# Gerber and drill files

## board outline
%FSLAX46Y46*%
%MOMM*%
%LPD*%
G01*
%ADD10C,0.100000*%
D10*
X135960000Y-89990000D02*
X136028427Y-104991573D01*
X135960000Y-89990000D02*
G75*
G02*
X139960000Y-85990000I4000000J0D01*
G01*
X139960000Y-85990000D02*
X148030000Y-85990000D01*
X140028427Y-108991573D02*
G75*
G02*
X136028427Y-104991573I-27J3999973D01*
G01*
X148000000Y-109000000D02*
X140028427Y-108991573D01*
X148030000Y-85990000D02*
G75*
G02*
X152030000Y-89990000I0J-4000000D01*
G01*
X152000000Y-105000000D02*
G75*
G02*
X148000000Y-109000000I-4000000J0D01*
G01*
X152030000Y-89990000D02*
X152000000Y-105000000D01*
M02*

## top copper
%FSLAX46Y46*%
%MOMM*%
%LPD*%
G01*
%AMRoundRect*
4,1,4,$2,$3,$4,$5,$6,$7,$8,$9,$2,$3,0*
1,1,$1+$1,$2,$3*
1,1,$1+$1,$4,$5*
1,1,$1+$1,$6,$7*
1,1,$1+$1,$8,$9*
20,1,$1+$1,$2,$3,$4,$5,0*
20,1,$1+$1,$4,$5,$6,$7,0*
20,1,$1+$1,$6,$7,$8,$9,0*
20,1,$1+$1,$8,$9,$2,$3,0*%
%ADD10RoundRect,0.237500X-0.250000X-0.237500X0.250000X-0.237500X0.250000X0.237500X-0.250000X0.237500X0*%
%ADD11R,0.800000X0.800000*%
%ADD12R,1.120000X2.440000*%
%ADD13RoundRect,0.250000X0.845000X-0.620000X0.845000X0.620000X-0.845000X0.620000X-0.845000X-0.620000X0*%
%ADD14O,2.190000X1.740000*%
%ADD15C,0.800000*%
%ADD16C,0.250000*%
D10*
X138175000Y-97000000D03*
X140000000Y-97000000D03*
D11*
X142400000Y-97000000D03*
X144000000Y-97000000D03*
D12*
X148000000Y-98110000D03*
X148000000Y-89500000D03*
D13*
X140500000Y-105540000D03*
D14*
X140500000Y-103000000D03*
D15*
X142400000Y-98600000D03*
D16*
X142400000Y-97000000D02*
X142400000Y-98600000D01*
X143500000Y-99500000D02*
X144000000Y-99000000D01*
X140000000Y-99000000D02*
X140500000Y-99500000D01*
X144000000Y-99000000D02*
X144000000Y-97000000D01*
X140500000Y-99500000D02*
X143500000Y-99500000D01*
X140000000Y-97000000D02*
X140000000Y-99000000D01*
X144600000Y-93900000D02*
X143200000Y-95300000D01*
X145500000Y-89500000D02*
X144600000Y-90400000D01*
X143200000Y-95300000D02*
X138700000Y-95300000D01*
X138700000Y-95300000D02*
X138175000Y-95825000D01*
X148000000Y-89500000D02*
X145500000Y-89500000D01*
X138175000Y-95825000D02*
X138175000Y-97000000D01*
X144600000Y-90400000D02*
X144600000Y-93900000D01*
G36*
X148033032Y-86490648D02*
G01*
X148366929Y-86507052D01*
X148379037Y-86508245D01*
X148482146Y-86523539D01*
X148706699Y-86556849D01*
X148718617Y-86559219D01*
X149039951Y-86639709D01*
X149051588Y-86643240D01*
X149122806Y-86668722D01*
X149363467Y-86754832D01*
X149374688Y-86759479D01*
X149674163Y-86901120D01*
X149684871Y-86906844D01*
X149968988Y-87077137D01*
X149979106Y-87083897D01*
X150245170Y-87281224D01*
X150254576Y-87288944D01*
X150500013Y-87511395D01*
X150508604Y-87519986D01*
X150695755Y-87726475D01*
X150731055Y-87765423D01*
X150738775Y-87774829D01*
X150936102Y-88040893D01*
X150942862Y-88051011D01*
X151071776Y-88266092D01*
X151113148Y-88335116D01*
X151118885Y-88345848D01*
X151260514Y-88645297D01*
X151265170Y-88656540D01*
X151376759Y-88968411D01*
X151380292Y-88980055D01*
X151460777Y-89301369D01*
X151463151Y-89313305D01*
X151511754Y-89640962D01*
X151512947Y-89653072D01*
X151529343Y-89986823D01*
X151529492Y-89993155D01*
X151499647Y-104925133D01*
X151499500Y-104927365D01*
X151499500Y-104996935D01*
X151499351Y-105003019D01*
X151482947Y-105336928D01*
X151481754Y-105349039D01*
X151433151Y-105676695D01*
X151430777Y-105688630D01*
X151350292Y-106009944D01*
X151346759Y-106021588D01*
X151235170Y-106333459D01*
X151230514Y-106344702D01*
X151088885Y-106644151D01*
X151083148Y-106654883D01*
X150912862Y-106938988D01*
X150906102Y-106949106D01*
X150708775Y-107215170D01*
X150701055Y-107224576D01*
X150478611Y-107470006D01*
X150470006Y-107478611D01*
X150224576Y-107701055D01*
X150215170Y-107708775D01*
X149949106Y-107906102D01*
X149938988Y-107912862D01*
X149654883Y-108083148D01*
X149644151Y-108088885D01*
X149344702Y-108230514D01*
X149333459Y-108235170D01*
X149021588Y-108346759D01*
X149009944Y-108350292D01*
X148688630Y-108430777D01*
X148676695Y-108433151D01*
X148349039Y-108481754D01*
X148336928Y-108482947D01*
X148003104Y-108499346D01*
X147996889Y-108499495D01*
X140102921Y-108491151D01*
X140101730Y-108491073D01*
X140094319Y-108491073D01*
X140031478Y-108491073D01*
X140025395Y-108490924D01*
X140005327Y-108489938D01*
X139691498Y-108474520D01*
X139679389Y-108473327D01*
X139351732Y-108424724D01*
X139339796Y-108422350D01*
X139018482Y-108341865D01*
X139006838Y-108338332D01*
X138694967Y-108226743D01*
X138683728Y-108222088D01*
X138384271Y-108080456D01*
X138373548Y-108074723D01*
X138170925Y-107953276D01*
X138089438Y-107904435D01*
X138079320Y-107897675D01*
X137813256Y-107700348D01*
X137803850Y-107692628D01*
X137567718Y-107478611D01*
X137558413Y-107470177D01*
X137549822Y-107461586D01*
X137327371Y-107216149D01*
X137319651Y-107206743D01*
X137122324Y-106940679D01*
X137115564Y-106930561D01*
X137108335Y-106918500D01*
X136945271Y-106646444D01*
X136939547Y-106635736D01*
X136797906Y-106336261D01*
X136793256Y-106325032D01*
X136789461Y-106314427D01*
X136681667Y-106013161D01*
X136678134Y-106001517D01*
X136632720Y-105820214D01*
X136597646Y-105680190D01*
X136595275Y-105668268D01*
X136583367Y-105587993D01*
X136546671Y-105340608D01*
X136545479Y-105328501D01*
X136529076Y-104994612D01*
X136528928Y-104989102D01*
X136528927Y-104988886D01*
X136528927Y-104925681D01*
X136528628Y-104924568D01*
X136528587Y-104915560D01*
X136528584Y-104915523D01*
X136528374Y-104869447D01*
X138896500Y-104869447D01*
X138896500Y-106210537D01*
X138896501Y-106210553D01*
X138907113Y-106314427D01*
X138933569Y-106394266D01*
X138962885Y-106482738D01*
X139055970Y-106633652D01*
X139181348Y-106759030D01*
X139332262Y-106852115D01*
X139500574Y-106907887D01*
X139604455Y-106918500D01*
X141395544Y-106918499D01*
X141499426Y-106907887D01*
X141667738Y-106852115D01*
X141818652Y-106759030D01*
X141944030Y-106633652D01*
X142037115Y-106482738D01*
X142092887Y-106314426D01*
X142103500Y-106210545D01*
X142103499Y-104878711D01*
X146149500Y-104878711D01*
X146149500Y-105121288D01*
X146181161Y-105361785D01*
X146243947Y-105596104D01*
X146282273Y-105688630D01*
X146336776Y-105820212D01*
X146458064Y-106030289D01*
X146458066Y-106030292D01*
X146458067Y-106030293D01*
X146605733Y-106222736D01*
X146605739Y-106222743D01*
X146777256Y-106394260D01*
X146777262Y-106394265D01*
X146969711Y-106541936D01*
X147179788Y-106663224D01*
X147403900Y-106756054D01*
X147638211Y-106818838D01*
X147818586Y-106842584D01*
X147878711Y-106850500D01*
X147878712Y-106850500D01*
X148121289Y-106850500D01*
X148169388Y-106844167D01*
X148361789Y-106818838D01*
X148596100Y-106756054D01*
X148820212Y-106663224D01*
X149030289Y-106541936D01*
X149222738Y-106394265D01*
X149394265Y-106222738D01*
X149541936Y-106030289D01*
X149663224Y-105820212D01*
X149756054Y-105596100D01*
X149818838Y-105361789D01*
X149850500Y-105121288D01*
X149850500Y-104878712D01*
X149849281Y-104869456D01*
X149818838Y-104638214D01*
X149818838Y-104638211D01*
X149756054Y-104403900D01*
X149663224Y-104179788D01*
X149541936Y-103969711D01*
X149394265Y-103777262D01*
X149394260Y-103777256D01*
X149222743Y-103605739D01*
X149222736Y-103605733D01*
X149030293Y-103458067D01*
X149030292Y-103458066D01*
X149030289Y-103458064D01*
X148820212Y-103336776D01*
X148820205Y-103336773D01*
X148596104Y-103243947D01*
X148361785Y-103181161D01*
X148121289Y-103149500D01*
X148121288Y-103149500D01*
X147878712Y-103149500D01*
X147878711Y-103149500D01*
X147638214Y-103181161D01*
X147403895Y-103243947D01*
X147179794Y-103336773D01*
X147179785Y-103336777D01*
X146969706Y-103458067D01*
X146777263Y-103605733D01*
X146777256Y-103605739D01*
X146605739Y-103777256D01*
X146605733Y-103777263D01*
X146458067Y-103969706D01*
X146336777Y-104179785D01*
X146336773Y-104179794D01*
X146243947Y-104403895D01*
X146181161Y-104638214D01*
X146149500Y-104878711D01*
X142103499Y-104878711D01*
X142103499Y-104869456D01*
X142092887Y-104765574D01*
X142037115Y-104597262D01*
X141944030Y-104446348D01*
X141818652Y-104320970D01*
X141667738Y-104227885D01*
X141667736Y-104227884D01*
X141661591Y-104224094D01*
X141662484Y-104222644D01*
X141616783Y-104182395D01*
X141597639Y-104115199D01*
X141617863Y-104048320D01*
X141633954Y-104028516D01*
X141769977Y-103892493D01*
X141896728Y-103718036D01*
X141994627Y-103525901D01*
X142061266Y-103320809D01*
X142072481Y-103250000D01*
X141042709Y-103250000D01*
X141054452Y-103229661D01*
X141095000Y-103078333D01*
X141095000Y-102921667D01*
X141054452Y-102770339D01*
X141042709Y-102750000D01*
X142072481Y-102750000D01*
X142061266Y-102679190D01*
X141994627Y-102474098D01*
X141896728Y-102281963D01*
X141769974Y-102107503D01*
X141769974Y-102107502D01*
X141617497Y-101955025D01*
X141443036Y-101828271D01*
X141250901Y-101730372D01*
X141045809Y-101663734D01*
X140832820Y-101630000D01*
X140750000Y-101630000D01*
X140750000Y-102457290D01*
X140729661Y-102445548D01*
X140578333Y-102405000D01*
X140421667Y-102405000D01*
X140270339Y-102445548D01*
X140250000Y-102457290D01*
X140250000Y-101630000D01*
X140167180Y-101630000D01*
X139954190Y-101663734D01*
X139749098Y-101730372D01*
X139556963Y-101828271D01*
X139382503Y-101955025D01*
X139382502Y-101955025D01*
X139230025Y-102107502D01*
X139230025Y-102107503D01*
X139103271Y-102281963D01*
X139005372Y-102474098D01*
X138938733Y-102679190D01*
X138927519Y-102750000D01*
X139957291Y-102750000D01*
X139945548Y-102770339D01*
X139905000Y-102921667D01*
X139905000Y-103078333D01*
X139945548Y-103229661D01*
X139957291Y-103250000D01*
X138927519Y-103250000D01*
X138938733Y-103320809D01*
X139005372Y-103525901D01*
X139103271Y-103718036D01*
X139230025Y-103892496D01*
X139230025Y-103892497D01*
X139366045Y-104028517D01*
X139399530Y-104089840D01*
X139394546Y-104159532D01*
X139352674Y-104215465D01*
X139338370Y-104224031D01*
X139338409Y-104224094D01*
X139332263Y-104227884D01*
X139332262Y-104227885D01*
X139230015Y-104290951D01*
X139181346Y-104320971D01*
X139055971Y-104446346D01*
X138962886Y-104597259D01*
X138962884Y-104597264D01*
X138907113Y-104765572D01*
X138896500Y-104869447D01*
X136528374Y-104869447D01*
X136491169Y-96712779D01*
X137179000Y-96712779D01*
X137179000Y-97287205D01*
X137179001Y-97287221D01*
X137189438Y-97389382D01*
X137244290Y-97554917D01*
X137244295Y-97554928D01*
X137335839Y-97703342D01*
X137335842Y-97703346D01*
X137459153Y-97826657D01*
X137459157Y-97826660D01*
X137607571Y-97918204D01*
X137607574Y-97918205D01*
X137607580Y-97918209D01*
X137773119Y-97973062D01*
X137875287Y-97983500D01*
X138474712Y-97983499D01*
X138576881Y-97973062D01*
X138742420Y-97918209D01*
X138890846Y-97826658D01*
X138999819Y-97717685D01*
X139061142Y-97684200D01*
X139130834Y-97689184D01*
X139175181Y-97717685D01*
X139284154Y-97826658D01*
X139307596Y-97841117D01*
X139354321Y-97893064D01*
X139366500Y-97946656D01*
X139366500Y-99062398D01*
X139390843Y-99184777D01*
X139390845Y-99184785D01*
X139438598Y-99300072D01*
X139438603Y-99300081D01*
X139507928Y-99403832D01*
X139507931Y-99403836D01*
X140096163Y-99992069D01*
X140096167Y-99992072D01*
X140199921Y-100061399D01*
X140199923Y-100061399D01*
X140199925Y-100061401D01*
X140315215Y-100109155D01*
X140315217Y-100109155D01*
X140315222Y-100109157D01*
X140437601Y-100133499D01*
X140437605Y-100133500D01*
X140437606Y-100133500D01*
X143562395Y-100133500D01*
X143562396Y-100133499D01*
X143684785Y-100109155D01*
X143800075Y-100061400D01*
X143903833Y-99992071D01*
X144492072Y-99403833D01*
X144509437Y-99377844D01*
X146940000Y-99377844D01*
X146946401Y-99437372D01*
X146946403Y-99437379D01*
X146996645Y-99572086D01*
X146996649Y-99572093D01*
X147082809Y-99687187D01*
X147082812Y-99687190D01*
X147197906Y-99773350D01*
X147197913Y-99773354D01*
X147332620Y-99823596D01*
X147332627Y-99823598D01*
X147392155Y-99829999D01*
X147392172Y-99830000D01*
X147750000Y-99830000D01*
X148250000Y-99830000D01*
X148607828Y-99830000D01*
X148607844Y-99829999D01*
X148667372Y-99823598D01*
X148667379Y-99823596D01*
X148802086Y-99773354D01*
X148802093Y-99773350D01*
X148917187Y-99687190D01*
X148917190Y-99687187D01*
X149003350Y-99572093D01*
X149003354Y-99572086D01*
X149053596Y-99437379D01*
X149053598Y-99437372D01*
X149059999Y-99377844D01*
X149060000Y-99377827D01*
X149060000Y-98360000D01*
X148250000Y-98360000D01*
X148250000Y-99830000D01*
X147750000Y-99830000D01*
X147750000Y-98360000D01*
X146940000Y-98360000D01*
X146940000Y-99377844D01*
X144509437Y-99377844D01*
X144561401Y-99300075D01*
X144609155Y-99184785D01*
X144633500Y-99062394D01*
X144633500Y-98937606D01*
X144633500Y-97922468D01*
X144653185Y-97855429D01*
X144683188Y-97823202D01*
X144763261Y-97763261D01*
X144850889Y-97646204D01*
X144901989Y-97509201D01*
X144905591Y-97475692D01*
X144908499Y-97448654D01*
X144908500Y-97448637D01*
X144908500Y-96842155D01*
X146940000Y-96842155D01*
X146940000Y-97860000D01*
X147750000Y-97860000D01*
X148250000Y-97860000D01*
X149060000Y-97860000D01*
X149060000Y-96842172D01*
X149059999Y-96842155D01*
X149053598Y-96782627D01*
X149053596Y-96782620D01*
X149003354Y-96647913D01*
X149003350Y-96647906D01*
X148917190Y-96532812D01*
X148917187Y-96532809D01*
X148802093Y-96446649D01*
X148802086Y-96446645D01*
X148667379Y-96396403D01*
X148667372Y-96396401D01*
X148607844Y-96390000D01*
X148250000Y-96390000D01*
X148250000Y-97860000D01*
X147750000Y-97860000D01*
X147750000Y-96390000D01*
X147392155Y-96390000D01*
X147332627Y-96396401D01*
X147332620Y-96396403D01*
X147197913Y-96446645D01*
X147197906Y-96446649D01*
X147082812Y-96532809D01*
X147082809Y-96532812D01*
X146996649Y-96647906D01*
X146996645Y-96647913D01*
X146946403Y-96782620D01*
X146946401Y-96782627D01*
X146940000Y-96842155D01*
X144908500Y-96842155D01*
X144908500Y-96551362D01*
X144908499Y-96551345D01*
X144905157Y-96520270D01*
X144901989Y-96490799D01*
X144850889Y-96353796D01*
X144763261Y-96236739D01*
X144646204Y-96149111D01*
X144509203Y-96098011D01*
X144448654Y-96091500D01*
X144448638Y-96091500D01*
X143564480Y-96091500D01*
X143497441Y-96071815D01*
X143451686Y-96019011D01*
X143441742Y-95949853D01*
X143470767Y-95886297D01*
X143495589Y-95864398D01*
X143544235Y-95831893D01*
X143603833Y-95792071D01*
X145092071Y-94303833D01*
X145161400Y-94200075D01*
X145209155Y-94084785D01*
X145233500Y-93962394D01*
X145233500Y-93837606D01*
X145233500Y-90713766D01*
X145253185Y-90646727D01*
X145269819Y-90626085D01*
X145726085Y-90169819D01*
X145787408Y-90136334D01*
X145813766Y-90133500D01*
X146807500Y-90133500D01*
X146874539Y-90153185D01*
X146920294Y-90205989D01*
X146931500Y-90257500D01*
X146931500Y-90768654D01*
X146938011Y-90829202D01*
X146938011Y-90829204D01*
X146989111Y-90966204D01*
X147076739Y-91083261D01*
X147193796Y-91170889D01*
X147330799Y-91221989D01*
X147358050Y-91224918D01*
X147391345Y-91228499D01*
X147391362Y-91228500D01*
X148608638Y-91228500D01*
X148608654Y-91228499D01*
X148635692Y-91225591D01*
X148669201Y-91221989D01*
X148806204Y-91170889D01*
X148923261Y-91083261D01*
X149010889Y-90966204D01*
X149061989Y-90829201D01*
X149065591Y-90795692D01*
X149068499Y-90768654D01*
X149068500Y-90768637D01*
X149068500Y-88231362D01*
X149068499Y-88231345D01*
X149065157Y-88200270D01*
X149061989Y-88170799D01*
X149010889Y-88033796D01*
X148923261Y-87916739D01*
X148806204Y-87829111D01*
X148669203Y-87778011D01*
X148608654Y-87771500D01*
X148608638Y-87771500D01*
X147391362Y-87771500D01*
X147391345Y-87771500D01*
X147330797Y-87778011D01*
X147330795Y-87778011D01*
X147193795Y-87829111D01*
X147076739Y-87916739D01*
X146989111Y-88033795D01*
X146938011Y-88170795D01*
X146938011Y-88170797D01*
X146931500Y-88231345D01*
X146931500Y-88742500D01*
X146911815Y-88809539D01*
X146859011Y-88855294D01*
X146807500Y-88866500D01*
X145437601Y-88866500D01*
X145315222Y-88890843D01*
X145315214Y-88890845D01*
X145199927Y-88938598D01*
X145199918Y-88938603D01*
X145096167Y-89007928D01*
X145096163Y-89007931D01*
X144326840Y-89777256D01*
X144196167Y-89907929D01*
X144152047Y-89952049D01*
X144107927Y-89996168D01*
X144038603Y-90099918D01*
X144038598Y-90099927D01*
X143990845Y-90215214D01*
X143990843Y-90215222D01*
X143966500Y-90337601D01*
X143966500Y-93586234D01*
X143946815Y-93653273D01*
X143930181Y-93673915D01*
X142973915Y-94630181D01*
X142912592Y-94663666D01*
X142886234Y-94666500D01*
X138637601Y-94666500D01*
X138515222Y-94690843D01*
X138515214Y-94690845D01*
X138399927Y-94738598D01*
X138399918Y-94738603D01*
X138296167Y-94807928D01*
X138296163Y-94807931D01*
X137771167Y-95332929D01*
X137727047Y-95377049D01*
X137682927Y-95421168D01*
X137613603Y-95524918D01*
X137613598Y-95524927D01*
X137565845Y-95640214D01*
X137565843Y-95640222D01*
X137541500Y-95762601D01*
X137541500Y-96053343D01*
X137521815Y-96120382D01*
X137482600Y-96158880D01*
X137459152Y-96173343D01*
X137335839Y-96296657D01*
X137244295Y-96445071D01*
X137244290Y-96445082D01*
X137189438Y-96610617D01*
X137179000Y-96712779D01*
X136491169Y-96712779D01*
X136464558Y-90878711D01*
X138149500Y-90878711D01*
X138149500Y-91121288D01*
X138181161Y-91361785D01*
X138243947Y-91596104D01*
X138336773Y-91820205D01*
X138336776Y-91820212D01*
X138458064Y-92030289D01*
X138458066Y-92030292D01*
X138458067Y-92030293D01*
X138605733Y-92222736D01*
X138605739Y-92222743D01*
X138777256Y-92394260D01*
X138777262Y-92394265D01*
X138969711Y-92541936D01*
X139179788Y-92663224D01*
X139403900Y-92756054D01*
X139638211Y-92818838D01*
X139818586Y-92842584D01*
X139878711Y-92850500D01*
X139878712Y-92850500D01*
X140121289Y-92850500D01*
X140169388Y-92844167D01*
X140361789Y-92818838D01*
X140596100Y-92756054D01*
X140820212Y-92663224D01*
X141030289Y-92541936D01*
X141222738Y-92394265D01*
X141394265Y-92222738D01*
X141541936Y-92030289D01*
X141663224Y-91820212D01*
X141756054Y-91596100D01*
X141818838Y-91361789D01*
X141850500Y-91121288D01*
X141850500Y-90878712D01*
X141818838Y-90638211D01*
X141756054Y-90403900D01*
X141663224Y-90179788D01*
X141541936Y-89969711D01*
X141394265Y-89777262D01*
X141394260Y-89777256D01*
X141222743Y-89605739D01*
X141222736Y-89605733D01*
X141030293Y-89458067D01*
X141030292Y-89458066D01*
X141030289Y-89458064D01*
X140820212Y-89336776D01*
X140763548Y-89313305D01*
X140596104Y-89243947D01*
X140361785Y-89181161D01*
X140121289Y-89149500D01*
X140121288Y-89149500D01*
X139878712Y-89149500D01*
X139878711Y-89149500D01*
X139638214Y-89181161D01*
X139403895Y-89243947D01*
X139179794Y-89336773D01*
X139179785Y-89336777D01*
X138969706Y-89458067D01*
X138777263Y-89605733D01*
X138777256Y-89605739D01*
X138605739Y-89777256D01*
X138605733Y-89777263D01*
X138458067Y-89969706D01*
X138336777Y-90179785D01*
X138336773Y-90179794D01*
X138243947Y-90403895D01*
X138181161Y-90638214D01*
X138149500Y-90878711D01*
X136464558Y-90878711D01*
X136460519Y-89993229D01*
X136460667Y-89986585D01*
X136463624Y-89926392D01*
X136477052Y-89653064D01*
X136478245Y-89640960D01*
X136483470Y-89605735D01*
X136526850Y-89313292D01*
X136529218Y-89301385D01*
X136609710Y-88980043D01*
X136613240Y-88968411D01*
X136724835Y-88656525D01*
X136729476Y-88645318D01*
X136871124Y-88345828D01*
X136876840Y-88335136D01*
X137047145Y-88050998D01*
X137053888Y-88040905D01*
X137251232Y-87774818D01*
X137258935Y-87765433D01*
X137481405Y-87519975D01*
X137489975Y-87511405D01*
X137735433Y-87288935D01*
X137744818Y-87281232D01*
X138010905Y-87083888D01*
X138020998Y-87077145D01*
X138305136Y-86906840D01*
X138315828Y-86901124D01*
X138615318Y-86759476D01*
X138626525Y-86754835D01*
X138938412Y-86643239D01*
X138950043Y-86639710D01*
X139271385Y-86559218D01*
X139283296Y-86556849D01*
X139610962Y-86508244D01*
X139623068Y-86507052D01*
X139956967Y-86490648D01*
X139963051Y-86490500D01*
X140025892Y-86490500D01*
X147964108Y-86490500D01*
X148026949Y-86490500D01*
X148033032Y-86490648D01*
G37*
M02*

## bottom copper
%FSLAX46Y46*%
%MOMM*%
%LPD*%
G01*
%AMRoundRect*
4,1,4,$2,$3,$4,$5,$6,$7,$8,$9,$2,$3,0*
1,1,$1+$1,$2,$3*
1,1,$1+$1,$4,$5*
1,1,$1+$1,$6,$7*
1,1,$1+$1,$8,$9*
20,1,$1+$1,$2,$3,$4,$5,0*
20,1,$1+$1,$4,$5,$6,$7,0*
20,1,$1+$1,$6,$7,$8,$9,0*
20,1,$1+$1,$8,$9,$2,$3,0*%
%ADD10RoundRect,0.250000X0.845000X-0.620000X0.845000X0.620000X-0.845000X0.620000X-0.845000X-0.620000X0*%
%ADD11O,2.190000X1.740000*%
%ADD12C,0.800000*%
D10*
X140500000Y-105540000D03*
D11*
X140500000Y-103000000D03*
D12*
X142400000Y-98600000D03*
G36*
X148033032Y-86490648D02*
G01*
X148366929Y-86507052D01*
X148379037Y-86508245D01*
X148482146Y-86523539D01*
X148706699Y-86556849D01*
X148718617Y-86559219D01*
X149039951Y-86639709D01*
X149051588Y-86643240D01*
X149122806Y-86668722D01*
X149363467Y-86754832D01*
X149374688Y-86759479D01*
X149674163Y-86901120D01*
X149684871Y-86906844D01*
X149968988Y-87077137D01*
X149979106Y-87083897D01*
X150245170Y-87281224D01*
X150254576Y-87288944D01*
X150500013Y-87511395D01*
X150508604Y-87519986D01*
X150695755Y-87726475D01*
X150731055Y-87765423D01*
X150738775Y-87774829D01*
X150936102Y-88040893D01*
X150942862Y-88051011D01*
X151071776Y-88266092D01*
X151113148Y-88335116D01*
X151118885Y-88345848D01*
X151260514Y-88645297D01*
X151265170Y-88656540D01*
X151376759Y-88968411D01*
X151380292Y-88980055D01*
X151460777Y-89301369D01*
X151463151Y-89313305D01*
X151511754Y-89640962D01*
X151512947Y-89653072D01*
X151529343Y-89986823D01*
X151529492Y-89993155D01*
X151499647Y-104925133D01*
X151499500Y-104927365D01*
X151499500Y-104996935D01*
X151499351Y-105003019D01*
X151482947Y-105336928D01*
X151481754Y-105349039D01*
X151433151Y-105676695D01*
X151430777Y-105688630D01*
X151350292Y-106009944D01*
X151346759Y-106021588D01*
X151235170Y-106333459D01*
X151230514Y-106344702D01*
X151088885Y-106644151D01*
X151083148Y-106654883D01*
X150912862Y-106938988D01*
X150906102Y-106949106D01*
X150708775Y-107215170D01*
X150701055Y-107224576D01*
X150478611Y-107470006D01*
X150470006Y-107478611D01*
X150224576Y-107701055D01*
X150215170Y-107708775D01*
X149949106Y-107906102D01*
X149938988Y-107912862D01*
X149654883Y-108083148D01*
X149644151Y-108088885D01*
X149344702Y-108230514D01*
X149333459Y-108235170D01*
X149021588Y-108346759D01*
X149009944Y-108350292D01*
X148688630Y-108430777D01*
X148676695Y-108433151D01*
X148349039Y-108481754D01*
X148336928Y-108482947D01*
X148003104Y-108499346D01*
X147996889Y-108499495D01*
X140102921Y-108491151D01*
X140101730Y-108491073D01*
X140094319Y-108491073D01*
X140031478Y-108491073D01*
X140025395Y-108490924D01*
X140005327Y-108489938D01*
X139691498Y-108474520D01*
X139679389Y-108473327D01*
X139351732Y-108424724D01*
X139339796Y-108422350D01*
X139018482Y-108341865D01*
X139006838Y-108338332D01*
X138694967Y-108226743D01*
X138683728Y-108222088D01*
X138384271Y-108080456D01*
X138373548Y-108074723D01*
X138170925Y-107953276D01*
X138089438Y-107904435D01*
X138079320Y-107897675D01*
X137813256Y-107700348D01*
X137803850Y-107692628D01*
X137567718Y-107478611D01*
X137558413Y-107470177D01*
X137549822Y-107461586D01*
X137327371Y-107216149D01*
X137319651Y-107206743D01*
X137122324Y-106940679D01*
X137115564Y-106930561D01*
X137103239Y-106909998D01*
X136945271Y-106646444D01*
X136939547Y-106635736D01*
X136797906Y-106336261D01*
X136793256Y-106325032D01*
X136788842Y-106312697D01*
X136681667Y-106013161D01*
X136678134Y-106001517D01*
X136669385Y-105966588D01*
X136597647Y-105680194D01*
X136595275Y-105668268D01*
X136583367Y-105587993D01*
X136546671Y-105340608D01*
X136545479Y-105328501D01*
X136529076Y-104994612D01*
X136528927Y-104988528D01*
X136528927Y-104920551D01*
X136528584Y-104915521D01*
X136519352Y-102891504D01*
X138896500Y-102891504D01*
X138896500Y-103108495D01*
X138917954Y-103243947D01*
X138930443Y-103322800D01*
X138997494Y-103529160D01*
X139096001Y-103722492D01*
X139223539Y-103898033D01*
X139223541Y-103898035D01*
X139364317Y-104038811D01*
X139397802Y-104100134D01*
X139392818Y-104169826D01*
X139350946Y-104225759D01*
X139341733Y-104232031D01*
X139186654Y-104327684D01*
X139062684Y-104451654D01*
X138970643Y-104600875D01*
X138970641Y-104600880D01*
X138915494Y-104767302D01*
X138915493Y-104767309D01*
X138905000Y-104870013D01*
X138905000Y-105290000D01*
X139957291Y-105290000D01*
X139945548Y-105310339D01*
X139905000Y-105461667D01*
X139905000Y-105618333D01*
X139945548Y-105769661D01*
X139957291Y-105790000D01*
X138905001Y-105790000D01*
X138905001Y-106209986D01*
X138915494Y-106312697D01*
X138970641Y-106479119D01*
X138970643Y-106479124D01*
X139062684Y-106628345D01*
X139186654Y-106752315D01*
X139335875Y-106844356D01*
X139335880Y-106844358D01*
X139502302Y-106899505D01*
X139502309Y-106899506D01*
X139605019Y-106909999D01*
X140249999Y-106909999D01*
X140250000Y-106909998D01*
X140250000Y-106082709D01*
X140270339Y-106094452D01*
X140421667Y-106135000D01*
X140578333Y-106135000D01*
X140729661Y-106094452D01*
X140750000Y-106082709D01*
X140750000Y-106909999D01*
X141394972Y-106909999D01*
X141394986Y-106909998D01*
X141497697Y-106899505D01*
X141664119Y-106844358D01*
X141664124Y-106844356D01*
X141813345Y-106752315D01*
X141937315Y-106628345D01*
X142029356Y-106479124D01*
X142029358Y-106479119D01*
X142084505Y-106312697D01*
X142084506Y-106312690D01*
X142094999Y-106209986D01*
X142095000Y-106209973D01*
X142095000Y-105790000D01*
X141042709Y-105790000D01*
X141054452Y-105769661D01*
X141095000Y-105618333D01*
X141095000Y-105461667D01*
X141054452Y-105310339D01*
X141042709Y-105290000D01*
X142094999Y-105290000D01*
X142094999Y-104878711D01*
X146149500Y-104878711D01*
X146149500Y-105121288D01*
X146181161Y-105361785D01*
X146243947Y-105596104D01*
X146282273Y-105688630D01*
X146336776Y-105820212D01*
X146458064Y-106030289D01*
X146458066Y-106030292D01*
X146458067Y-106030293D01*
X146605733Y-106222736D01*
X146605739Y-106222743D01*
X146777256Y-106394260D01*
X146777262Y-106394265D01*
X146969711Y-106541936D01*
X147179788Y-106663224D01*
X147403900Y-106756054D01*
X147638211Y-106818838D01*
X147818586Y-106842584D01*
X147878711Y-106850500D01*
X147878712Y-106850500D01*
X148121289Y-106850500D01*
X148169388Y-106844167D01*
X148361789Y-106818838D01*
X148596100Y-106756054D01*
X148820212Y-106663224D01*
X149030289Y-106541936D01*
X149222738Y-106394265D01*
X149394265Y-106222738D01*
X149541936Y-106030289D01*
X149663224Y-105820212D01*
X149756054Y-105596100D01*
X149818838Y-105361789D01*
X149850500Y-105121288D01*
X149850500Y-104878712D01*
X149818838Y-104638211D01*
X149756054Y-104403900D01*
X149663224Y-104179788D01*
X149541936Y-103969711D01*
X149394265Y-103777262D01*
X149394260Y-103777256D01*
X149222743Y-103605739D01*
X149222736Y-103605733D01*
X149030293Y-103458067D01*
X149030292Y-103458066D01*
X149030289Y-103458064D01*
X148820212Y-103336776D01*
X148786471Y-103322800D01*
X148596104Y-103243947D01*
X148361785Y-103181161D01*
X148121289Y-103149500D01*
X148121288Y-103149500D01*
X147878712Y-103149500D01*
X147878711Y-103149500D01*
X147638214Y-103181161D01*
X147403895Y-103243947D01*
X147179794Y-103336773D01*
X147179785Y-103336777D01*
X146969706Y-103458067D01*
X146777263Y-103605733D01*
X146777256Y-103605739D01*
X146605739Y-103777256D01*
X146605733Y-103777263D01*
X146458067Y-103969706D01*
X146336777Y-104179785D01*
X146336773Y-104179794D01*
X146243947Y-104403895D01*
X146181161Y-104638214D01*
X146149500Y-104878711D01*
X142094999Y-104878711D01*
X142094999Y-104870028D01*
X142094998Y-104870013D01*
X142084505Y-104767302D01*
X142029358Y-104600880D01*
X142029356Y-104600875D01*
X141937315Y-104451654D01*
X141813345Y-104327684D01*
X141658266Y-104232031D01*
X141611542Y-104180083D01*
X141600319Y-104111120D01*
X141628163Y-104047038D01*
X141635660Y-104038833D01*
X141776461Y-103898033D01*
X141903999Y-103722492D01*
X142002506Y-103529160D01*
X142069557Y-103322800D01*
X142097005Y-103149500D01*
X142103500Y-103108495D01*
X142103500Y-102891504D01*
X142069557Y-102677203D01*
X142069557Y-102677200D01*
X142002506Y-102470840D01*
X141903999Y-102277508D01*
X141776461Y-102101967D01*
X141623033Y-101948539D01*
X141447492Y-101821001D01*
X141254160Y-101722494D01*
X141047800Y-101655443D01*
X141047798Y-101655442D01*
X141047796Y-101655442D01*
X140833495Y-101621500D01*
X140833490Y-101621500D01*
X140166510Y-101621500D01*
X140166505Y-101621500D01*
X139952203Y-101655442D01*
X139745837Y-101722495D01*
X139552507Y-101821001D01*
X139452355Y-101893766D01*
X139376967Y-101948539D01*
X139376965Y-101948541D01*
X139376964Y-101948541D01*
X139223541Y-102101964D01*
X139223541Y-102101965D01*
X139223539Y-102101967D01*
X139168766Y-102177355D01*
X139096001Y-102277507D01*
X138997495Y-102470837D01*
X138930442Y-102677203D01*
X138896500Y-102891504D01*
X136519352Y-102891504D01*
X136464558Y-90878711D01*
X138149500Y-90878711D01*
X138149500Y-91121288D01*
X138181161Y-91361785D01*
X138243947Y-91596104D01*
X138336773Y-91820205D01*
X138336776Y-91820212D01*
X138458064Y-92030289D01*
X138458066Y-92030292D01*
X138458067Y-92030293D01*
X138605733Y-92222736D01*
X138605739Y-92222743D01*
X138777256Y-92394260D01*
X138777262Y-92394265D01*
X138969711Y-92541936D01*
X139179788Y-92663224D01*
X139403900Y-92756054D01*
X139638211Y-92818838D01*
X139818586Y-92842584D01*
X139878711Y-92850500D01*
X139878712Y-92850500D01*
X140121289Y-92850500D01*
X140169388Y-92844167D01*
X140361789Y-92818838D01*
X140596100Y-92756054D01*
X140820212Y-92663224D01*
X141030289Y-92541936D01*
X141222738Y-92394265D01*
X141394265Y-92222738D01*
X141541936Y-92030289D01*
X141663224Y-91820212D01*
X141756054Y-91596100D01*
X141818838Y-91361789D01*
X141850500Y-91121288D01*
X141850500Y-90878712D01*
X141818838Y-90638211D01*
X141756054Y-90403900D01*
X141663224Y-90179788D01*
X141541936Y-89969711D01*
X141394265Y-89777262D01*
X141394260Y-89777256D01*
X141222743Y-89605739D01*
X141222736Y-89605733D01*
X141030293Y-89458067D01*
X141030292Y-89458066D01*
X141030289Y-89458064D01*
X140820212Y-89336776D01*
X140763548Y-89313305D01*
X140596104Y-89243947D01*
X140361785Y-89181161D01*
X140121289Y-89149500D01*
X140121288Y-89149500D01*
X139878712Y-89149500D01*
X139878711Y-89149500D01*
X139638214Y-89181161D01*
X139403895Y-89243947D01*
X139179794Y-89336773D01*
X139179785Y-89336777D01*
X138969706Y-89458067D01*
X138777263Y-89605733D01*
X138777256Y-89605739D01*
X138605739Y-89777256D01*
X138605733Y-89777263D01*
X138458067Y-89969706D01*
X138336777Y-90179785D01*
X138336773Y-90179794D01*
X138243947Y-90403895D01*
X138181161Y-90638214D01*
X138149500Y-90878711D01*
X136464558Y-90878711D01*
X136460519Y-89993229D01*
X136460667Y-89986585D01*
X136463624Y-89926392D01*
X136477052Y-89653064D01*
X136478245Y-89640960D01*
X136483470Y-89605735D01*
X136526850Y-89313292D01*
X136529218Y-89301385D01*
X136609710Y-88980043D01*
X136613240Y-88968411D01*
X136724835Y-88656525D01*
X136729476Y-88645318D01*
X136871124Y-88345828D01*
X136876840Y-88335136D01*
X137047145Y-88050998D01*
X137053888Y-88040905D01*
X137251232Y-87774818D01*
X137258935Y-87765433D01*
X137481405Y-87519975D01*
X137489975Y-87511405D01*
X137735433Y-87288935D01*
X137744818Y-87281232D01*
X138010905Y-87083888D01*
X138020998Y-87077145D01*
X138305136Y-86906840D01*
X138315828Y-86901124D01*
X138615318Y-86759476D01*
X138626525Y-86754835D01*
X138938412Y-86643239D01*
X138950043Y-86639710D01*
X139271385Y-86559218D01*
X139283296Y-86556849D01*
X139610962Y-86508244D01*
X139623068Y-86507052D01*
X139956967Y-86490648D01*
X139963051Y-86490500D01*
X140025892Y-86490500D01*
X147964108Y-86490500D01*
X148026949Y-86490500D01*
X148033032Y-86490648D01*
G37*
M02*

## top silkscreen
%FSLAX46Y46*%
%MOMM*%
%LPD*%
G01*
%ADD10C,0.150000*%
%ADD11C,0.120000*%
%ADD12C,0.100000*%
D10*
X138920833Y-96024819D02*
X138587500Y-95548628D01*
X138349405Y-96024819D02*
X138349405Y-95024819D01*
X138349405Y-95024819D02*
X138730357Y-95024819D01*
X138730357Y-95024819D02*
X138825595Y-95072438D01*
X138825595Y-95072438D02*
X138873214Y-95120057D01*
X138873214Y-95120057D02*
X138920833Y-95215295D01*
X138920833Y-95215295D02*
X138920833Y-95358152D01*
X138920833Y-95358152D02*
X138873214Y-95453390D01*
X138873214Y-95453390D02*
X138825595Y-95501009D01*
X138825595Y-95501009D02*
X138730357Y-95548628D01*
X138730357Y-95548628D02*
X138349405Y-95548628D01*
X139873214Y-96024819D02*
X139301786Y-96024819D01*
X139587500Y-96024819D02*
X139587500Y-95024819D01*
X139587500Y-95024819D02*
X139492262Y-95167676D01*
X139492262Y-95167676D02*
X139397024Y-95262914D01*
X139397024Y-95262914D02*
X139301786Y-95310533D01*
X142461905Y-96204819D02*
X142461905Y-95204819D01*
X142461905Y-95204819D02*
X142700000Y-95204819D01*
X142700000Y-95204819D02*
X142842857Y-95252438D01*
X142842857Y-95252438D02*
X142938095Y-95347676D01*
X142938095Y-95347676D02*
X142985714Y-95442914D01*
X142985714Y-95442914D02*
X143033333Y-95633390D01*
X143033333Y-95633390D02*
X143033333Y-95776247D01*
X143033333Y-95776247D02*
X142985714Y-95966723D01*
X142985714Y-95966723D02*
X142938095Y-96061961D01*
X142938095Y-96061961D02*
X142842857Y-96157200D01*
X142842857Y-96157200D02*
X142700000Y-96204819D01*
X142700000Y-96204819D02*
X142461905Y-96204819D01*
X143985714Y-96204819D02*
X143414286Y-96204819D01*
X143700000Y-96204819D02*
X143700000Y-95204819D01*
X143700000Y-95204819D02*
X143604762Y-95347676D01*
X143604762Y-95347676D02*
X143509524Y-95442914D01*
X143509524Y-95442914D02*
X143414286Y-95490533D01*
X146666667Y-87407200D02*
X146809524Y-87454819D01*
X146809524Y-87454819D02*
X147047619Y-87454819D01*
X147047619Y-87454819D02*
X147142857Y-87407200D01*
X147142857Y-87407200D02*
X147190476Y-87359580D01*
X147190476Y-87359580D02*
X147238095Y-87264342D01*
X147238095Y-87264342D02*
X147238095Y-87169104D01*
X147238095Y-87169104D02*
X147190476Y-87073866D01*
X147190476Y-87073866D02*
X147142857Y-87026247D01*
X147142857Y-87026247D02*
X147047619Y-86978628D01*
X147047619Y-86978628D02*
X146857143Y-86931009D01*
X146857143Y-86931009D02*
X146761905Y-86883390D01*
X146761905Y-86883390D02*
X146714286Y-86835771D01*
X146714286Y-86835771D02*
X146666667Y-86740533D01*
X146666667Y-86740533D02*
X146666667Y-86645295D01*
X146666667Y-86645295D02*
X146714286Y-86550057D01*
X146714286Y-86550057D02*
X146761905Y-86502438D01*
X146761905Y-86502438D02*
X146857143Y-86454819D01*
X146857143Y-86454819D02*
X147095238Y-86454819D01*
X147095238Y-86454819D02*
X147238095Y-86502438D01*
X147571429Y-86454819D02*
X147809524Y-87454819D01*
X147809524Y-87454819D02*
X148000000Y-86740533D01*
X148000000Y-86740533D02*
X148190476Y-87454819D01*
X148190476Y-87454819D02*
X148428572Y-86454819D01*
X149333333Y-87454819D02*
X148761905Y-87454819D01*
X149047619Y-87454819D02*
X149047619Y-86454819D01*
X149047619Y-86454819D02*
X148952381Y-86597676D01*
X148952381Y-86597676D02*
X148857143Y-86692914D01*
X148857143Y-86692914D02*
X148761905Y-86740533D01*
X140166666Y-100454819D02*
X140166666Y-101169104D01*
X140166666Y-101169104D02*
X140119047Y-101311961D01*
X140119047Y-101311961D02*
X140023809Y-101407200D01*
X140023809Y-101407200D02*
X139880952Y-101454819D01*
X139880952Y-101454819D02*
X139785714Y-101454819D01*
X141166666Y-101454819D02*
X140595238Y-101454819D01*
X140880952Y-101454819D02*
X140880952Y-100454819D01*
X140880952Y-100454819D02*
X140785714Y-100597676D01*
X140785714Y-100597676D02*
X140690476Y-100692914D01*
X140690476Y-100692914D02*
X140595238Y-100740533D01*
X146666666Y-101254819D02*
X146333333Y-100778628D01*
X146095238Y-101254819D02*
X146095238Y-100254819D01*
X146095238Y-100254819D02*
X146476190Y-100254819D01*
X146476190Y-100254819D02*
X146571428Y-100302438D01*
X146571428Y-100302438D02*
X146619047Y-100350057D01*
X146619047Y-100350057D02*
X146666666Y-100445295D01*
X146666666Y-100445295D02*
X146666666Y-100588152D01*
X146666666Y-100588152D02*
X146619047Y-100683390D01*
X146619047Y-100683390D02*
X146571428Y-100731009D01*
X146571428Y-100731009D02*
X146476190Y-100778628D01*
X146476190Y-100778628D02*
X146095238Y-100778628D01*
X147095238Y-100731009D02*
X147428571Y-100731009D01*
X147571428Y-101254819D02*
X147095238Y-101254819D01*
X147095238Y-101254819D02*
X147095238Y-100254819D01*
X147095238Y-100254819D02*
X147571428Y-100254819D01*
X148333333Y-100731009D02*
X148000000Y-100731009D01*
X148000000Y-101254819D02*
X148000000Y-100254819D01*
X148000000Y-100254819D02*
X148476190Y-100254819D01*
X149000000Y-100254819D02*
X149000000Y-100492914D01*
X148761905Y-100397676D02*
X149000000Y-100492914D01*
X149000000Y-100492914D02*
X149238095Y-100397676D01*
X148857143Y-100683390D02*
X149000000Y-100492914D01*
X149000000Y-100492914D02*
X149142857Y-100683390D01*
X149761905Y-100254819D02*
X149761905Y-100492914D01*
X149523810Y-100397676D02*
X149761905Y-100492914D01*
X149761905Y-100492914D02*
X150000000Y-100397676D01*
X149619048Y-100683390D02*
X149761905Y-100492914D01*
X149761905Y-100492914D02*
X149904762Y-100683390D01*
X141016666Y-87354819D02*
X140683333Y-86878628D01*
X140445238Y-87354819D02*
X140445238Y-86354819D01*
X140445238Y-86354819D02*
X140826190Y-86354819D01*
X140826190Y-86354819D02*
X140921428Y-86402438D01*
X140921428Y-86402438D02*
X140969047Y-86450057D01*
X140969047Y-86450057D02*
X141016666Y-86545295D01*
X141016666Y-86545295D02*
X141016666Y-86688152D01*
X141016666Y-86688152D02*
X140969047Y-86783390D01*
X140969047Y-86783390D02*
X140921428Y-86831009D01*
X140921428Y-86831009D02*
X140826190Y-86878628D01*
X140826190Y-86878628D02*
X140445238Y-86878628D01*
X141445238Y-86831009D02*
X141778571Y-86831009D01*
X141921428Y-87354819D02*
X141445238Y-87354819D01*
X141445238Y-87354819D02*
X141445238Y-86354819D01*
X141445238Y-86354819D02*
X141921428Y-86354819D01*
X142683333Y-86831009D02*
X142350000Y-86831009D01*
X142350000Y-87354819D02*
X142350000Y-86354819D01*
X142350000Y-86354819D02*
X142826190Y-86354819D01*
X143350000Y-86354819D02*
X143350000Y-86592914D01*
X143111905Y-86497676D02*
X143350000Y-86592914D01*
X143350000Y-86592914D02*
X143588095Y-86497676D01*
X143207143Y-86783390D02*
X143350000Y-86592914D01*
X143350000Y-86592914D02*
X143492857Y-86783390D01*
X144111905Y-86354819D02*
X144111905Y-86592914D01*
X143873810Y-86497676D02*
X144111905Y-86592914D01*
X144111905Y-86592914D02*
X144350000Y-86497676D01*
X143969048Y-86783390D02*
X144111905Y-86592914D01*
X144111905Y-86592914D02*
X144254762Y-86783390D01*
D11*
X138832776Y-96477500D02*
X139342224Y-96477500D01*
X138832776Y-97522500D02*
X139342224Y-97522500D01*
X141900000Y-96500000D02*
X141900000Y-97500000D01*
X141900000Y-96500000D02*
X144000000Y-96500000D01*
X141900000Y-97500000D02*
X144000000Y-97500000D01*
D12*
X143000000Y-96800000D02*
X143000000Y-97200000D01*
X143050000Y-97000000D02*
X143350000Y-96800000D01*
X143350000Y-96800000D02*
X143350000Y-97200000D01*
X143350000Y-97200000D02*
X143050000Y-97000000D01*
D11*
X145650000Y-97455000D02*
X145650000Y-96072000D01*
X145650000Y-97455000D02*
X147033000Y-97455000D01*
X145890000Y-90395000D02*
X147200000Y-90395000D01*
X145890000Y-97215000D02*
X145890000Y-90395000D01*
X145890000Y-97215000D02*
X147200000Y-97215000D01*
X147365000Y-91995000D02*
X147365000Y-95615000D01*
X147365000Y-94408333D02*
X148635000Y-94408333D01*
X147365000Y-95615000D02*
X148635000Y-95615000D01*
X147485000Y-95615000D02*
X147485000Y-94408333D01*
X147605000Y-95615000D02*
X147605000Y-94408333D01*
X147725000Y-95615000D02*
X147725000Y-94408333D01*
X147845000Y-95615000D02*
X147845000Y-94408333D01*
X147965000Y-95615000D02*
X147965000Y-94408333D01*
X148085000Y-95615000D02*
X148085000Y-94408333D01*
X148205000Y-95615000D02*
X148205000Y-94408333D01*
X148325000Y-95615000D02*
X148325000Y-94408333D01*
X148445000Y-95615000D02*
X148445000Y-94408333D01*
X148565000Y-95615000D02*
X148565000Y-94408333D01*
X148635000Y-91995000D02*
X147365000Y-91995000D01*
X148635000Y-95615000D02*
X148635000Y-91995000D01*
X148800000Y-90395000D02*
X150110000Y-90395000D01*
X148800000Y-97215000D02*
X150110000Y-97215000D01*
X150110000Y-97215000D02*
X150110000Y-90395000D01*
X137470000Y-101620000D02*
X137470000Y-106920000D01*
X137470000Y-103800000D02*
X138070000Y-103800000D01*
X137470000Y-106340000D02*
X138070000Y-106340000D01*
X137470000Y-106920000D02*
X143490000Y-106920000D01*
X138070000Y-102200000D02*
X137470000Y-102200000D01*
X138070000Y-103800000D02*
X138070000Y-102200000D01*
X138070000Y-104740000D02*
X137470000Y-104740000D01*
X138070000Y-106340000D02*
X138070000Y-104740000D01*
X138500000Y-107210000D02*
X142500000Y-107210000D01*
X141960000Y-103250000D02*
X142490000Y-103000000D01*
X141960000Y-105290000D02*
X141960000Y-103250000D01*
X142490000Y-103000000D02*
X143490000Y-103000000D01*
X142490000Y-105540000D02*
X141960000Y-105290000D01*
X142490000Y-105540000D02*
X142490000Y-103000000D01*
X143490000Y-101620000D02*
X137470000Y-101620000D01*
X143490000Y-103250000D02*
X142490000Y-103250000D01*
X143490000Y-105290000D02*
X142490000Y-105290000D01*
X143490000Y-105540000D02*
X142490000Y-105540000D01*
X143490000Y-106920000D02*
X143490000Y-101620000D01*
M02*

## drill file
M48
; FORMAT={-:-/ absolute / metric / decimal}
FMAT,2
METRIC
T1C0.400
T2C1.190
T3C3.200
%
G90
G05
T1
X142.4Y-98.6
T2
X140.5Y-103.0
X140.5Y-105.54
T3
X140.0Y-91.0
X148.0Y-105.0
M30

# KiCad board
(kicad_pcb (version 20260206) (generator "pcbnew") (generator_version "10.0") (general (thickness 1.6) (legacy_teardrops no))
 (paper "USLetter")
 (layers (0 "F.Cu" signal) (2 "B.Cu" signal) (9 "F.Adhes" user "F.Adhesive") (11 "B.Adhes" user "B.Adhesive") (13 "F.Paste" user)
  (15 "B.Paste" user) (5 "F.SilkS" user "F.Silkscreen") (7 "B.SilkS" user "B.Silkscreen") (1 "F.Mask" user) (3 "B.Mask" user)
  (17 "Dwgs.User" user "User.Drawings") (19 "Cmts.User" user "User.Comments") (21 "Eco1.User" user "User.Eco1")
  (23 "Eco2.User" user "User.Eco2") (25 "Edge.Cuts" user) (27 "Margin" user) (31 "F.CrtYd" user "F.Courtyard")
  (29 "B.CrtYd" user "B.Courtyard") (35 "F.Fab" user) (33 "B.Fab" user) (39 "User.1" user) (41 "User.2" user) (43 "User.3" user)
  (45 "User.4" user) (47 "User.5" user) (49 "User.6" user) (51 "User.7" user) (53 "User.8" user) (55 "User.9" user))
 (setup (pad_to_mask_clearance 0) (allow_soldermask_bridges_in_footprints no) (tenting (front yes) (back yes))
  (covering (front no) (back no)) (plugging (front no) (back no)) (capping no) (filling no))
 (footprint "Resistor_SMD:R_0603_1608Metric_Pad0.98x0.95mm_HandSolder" (layer "F.Cu") (at 139.0875 97)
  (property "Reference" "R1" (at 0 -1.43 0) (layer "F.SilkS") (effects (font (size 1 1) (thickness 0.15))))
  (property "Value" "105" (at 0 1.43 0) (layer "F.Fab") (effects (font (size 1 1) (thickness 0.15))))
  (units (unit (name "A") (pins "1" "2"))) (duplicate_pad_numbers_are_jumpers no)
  (fp_line (start -0.254724 -0.5225) (end 0.254724 -0.5225) (stroke (width 0.12) (type solid)) (layer "F.SilkS"))
  (fp_line (start -0.254724 0.5225) (end 0.254724 0.5225) (stroke (width 0.12) (type solid)) (layer "F.SilkS"))
  (pad "1" smd roundrect (at -0.9125 0) (size 0.975 0.95) (layers "F.Cu" "F.Mask" "F.Paste") (roundrect_rratio 0.25) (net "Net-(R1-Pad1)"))
  (pad "2" smd roundrect (at 0.9125 0) (size 0.975 0.95) (layers "F.Cu" "F.Mask" "F.Paste") (roundrect_rratio 0.25) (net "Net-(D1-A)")))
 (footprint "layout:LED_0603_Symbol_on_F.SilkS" (layer "F.Cu") (at 143.2 97)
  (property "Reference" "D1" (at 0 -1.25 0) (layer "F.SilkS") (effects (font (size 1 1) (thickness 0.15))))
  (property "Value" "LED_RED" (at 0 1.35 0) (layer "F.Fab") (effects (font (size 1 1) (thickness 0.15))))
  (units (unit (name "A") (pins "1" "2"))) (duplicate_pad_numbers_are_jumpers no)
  (fp_line (start -1.3 -0.5) (end -1.3 0.5) (stroke (width 0.12) (type solid)) (layer "F.SilkS"))
  (fp_line (start -1.3 -0.5) (end 0.8 -0.5) (stroke (width 0.12) (type solid)) (layer "F.SilkS"))
  (fp_line (start -1.3 0.5) (end 0.8 0.5) (stroke (width 0.12) (type solid)) (layer "F.SilkS"))
  (fp_line (start -0.2 -0.2) (end -0.2 0.2) (stroke (width 0.1) (type solid)) (layer "F.SilkS"))
  (fp_line (start -0.15 0) (end 0.15 -0.2) (stroke (width 0.1) (type solid)) (layer "F.SilkS"))
  (fp_line (start 0.15 -0.2) (end 0.15 0.2) (stroke (width 0.1) (type solid)) (layer "F.SilkS"))
  (fp_line (start 0.15 0.2) (end -0.15 0) (stroke (width 0.1) (type solid)) (layer "F.SilkS"))
  (pad "1" smd rect (at -0.8 0 180) (size 0.8 0.8) (layers "F.Cu" "F.Mask" "F.Paste") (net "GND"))
  (pad "2" smd rect (at 0.8 0 180) (size 0.8 0.8) (layers "F.Cu" "F.Mask" "F.Paste") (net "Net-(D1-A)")))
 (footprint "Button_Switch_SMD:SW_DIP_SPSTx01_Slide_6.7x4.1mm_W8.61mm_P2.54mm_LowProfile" (layer "F.Cu") (at 148 93.805 90)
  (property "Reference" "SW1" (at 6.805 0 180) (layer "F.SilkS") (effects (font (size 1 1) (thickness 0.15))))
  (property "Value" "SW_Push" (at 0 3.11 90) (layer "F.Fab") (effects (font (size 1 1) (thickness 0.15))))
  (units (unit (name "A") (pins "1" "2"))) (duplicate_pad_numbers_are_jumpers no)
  (fp_line (start -3.65 -2.35) (end -2.267 -2.35) (stroke (width 0.12) (type solid)) (layer "F.SilkS"))
  (fp_line (start -3.65 -2.35) (end -3.65 -0.967) (stroke (width 0.12) (type solid)) (layer "F.SilkS"))
  (fp_line (start 3.41 -2.11) (end 3.41 -0.8) (stroke (width 0.12) (type solid)) (layer "F.SilkS"))
  (fp_line (start -3.41 -2.11) (end 3.41 -2.11) (stroke (width 0.12) (type solid)) (layer "F.SilkS"))
  (fp_line (start -3.41 -2.11) (end -3.41 -0.8) (stroke (width 0.12) (type solid)) (layer "F.SilkS"))
  (fp_line (start 1.81 -0.635) (end -1.81 -0.635) (stroke (width 0.12) (type solid)) (layer "F.SilkS"))
  (fp_line (start -0.603333 -0.635) (end -0.603333 0.635) (stroke (width 0.12) (type solid)) (layer "F.SilkS"))
  (fp_line (start -1.81 -0.635) (end -1.81 0.635) (stroke (width 0.12) (type solid)) (layer "F.SilkS"))
  (fp_line (start -1.81 -0.515) (end -0.603333 -0.515) (stroke (width 0.12) (type solid)) (layer "F.SilkS"))
  (fp_line (start -1.81 -0.395) (end -0.603333 -0.395) (stroke (width 0.12) (type solid)) (layer "F.SilkS"))
  (fp_line (start -1.81 -0.275) (end -0.603333 -0.275) (stroke (width 0.12) (type solid)) (layer "F.SilkS"))
  (fp_line (start -1.81 -0.155) (end -0.603333 -0.155) (stroke (width 0.12) (type solid)) (layer "F.SilkS"))
  (fp_line (start -1.81 -0.035) (end -0.603333 -0.035) (stroke (width 0.12) (type solid)) (layer "F.SilkS"))
  (fp_line (start -1.81 0.085) (end -0.603333 0.085) (stroke (width 0.12) (type solid)) (layer "F.SilkS"))
  (fp_line (start -1.81 0.205) (end -0.603333 0.205) (stroke (width 0.12) (type solid)) (layer "F.SilkS"))
  (fp_line (start -1.81 0.325) (end -0.603333 0.325) (stroke (width 0.12) (type solid)) (layer "F.SilkS"))
  (fp_line (start -1.81 0.445) (end -0.603333 0.445) (stroke (width 0.12) (type solid)) (layer "F.SilkS"))
  (fp_line (start -1.81 0.565) (end -0.603333 0.565) (stroke (width 0.12) (type solid)) (layer "F.SilkS"))
  (fp_line (start 1.81 0.635) (end 1.81 -0.635) (stroke (width 0.12) (type solid)) (layer "F.SilkS"))
  (fp_line (start -1.81 0.635) (end 1.81 0.635) (stroke (width 0.12) (type solid)) (layer "F.SilkS"))
  (fp_line (start 3.41 0.8) (end 3.41 2.11) (stroke (width 0.12) (type solid)) (layer "F.SilkS"))
  (fp_line (start -3.41 0.8) (end -3.41 2.11) (stroke (width 0.12) (type solid)) (layer "F.SilkS"))
  (fp_line (start -3.41 2.11) (end 3.41 2.11) (stroke (width 0.12) (type solid)) (layer "F.SilkS"))
  (pad "1" smd rect (at -4.305 0 90) (size 2.44 1.12) (layers "F.Cu" "F.Mask" "F.Paste") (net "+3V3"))
  (pad "2" smd rect (at 4.305 0 90) (size 2.44 1.12) (layers "F.Cu" "F.Mask" "F.Paste") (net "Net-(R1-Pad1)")))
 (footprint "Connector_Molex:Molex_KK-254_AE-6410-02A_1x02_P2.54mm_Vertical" (layer "F.Cu") (at 140.5 105.54 90)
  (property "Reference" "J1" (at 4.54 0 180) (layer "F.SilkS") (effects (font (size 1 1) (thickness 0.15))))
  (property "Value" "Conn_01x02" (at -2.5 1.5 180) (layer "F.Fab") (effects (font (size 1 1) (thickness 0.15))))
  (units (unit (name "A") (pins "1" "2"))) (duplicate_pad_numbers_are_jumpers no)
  (fp_line (start 3.92 -3.03) (end -1.38 -3.03) (stroke (width 0.12) (type solid)) (layer "F.SilkS"))
  (fp_line (start 1.74 -3.03) (end 1.74 -2.43) (stroke (width 0.12) (type solid)) (layer "F.SilkS"))
  (fp_line (start -0.8 -3.03) (end -0.8 -2.43) (stroke (width 0.12) (type solid)) (layer "F.SilkS"))
  (fp_line (start -1.38 -3.03) (end -1.38 2.99) (stroke (width 0.12) (type solid)) (layer "F.SilkS"))
  (fp_line (start 3.34 -2.43) (end 3.34 -3.03) (stroke (width 0.12) (type solid)) (layer "F.SilkS"))
  (fp_line (start 1.74 -2.43) (end 3.34 -2.43) (stroke (width 0.12) (type solid)) (layer "F.SilkS"))
  (fp_line (start 0.8 -2.43) (end 0.8 -3.03) (stroke (width 0.12) (type solid)) (layer "F.SilkS"))
  (fp_line (start -0.8 -2.43) (end 0.8 -2.43) (stroke (width 0.12) (type solid)) (layer "F.SilkS"))
  (fp_line (start -1.67 -2) (end -1.67 2) (stroke (width 0.12) (type solid)) (layer "F.SilkS"))
  (fp_line (start 2.29 1.46) (end 2.54 1.99) (stroke (width 0.12) (type solid)) (layer "F.SilkS"))
  (fp_line (start 0.25 1.46) (end 2.29 1.46) (stroke (width 0.12) (type solid)) (layer "F.SilkS"))
  (fp_line (start 2.54 1.99) (end 2.54 2.99) (stroke (width 0.12) (type solid)) (layer "F.SilkS"))
  (fp_line (start 0 1.99) (end 0.25 1.46) (stroke (width 0.12) (type solid)) (layer "F.SilkS"))
  (fp_line (start 0 1.99) (end 2.54 1.99) (stroke (width 0.12) (type solid)) (layer "F.SilkS"))
  (fp_line (start 3.92 2.99) (end 3.92 -3.03) (stroke (width 0.12) (type solid)) (layer "F.SilkS"))
  (fp_line (start 2.29 2.99) (end 2.29 1.99) (stroke (width 0.12) (type solid)) (layer "F.SilkS"))
  (fp_line (start 0.25 2.99) (end 0.25 1.99) (stroke (width 0.12) (type solid)) (layer "F.SilkS"))
  (fp_line (start 0 2.99) (end 0 1.99) (stroke (width 0.12) (type solid)) (layer "F.SilkS"))
  (fp_line (start -1.38 2.99) (end 3.92 2.99) (stroke (width 0.12) (type solid)) (layer "F.SilkS"))
  (pad "1" thru_hole roundrect (at 0 0 90) (size 1.74 2.19) (drill 1.19) (layers "*.Cu" "*.Mask") (remove_unused_layers no)
   (roundrect_rratio 0.143678) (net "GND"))
  (pad "2" thru_hole oval (at 2.54 0 90) (size 1.74 2.19) (drill 1.19) (layers "*.Cu" "*.Mask") (remove_unused_layers no) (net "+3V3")))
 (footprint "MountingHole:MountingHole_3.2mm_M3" (layer "F.Cu") (at 148 105)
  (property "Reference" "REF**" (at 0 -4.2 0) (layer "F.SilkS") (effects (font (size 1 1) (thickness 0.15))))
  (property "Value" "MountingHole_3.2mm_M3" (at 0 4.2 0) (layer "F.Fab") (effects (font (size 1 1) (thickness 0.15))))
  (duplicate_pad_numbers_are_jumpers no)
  (pad "" np_thru_hole circle (at 0 0) (size 3.2 3.2) (drill 3.2) (layers "*.Cu" "*.Mask")))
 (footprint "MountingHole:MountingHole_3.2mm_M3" (layer "F.Cu") (at 140 91)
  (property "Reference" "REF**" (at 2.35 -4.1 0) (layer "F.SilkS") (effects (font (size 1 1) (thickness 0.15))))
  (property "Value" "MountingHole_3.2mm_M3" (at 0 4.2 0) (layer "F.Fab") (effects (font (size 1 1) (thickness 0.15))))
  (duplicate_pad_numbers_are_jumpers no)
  (pad "" np_thru_hole circle (at 0 0) (size 3.2 3.2) (drill 3.2) (layers "*.Cu" "*.Mask")))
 (gr_line (start 135.96 89.99) (end 136.028427 104.991573) (stroke (width 0.1) (type default)) (layer "Edge.Cuts"))
 (gr_arc (start 135.96 89.99) (mid 137.131573 87.161573) (end 139.96 85.99) (stroke (width 0.1) (type default)) (layer "Edge.Cuts"))
 (gr_line (start 139.96 85.99) (end 148.03 85.99) (stroke (width 0.1) (type default)) (layer "Edge.Cuts"))
 (gr_arc (start 140.028427 108.991573) (mid 137.2 107.82) (end 136.028427 104.991573) (stroke (width 0.1) (type default))
  (layer "Edge.Cuts"))
 (gr_line (start 148 109) (end 140.028427 108.991573) (stroke (width 0.1) (type default)) (layer "Edge.Cuts"))
 (gr_arc (start 148.03 85.99) (mid 150.858427 87.161573) (end 152.03 89.99) (stroke (width 0.1) (type default)) (layer "Edge.Cuts"))
 (gr_arc (start 152 105) (mid 150.828427 107.828427) (end 148 109) (stroke (width 0.1) (type default)) (layer "Edge.Cuts"))
 (gr_line (start 152.03 89.99) (end 152 105) (stroke (width 0.1) (type default)) (layer "Edge.Cuts"))
 (segment (start 142.4 97) (end 142.4 98.6) (width 0.25) (layer "F.Cu") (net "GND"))
 (via (at 142.4 98.6) (size 0.8) (drill 0.4) (layers "F.Cu" "B.Cu") (free yes) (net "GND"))
 (segment (start 143.5 99.5) (end 144 99) (width 0.25) (layer "F.Cu") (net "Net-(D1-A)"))
 (segment (start 140 99) (end 140.5 99.5) (width 0.25) (layer "F.Cu") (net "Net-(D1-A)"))
 (segment (start 144 99) (end 144 97) (width 0.25) (layer "F.Cu") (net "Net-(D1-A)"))
 (segment (start 140.5 99.5) (end 143.5 99.5) (width 0.25) (layer "F.Cu") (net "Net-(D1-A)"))
 (segment (start 140 97) (end 140 99) (width 0.25) (layer "F.Cu") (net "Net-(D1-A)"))
 (segment (start 144.6 93.9) (end 143.2 95.3) (width 0.25) (layer "F.Cu") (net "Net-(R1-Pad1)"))
 (segment (start 145.5 89.5) (end 144.6 90.4) (width 0.25) (layer "F.Cu") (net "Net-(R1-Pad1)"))
 (segment (start 143.2 95.3) (end 138.7 95.3) (width 0.25) (layer "F.Cu") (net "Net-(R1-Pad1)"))
 (segment (start 138.7 95.3) (end 138.175 95.825) (width 0.25) (layer "F.Cu") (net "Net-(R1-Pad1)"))
 (segment (start 148 89.5) (end 145.5 89.5) (width 0.25) (layer "F.Cu") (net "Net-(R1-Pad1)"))
 (segment (start 138.175 95.825) (end 138.175 97) (width 0.25) (layer "F.Cu") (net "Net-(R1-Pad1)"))
 (segment (start 144.6 90.4) (end 144.6 93.9) (width 0.25) (layer "F.Cu") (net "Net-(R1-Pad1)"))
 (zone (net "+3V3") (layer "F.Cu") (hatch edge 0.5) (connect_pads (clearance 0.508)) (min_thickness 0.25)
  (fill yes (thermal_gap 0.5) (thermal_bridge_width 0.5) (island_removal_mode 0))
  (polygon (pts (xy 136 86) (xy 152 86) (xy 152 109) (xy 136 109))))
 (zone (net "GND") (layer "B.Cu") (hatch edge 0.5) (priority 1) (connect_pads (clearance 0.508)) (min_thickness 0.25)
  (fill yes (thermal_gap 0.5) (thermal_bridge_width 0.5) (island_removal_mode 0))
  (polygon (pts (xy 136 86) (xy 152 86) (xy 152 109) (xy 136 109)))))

